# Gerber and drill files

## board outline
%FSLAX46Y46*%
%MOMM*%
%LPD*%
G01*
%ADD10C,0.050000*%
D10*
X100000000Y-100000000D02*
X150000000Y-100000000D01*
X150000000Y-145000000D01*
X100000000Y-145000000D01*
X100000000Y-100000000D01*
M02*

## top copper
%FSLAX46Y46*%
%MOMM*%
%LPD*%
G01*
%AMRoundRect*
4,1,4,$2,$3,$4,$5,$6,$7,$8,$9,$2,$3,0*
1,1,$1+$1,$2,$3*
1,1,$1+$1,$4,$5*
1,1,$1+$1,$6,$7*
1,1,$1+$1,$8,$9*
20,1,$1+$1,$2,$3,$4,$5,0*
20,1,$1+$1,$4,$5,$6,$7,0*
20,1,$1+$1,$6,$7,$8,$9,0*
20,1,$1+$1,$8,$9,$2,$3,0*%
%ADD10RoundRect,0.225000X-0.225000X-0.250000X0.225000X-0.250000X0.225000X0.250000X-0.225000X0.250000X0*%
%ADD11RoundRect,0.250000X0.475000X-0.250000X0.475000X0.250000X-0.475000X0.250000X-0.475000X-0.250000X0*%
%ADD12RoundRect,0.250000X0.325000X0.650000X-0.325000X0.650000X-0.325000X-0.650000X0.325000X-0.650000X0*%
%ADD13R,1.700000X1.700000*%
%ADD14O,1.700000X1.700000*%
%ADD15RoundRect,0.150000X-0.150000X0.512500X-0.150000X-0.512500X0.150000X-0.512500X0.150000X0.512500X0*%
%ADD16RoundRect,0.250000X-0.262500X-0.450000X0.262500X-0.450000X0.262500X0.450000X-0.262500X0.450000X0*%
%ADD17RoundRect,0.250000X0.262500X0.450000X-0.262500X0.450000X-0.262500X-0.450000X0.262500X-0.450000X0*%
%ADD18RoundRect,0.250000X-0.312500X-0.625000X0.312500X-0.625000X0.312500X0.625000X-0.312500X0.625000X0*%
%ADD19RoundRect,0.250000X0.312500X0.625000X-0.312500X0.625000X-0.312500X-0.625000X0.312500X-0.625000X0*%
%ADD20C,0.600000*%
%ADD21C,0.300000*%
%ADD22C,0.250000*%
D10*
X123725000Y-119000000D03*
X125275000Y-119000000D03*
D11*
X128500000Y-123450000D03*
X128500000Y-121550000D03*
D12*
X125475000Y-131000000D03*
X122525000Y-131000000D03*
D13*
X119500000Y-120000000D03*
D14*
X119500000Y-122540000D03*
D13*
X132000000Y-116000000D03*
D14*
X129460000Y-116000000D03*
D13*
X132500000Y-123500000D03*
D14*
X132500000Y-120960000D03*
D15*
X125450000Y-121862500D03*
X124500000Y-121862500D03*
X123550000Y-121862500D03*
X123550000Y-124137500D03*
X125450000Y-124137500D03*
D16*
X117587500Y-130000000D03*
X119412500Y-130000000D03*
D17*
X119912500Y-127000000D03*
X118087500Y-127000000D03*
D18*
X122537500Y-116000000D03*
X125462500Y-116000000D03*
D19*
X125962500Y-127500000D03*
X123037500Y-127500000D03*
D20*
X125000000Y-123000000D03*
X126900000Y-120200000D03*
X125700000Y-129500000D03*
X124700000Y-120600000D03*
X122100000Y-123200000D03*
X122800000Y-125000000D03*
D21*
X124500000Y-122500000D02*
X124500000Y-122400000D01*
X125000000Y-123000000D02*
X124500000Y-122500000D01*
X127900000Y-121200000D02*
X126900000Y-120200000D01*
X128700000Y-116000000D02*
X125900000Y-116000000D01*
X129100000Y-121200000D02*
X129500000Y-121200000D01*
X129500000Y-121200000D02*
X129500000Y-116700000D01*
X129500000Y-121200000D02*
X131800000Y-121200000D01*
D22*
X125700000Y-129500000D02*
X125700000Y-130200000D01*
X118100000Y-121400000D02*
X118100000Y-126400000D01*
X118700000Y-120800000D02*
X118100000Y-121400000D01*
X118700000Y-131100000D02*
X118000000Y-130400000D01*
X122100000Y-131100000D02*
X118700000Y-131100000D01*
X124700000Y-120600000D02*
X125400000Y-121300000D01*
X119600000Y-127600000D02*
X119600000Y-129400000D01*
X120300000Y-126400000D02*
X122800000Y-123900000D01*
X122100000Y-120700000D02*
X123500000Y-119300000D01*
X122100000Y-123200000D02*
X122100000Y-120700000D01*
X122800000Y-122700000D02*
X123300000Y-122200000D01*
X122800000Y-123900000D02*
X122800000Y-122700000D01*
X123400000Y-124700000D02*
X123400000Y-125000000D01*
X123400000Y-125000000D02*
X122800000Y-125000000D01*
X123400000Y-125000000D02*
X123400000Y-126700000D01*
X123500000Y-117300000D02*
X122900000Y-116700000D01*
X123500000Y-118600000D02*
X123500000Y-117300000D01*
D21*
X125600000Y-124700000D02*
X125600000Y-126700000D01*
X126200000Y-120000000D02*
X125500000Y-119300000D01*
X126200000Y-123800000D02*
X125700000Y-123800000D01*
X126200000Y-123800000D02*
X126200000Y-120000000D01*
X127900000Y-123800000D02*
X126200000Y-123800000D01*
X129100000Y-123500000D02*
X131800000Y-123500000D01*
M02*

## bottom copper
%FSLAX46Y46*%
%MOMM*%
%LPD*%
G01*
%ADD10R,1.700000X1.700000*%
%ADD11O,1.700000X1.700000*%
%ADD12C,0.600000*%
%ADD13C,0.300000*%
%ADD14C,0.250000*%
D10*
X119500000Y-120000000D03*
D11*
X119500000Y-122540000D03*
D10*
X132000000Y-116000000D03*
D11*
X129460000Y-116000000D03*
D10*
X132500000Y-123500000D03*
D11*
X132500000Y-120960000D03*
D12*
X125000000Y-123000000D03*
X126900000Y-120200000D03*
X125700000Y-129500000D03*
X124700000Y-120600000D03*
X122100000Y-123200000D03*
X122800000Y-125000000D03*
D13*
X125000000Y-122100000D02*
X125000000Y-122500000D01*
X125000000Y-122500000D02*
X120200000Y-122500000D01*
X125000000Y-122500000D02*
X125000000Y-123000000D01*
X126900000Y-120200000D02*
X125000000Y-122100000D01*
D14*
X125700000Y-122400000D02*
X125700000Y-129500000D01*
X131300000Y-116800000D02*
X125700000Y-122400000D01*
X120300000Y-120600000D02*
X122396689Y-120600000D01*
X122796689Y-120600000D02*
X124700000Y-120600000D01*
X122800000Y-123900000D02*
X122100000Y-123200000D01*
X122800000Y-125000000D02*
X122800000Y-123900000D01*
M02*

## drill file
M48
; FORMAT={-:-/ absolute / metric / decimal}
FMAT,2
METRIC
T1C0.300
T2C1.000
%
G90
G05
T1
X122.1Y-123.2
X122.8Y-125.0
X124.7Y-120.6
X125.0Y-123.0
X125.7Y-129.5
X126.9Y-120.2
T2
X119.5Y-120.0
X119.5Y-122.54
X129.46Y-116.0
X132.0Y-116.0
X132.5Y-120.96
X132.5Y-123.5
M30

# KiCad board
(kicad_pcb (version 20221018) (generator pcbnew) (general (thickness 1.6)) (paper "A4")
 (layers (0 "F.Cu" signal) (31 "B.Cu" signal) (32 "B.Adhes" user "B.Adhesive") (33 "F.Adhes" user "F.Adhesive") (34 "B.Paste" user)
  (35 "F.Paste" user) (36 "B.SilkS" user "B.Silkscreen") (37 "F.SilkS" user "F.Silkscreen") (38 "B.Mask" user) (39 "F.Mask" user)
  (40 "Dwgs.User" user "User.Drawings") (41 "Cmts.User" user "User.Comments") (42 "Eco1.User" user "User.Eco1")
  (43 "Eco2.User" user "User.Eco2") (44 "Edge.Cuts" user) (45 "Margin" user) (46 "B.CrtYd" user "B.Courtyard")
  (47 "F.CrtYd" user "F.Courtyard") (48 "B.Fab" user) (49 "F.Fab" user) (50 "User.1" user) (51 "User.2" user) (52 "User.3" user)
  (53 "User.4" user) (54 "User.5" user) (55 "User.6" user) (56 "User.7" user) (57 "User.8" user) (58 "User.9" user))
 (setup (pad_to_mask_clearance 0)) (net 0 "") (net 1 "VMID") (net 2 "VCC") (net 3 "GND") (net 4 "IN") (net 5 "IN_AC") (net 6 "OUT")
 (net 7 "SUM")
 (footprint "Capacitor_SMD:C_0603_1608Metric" (layer "F.Cu") (at 124.5 119)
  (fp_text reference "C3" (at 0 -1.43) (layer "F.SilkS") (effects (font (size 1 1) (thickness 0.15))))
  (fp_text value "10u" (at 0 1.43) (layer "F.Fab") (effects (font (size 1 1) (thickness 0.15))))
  (pad "1" smd roundrect (at -0.775 0) (size 0.9 0.95) (layers "F.Cu" "F.Paste" "F.Mask") (roundrect_rratio 0.25) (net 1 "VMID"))
  (pad "2" smd roundrect (at 0.775 0) (size 0.9 0.95) (layers "F.Cu" "F.Paste" "F.Mask") (roundrect_rratio 0.25) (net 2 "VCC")))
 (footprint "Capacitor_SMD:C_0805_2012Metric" (layer "F.Cu") (at 128.5 122.5 90)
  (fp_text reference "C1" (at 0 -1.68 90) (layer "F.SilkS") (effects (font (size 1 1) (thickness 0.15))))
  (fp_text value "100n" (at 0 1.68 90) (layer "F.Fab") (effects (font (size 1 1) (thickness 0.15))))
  (pad "1" smd roundrect (at -0.95 0 90) (size 1 1.45) (layers "F.Cu" "F.Paste" "F.Mask") (roundrect_rratio 0.25) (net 2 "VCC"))
  (pad "2" smd roundrect (at 0.95 0 90) (size 1 1.45) (layers "F.Cu" "F.Paste" "F.Mask") (roundrect_rratio 0.25) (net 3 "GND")))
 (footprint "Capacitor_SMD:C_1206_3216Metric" (layer "F.Cu") (at 124 131 180)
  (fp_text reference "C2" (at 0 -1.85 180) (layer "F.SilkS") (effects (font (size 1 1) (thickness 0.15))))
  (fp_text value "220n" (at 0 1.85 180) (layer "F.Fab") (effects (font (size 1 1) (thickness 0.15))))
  (pad "1" smd roundrect (at -1.475 0 180) (size 1.15 1.8) (layers "F.Cu" "F.Paste" "F.Mask") (roundrect_rratio 0.217391) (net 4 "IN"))
  (pad "2" smd roundrect (at 1.475 0 180) (size 1.15 1.8) (layers "F.Cu" "F.Paste" "F.Mask") (roundrect_rratio 0.217391) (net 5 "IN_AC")))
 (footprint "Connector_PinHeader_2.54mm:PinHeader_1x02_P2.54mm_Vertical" (layer "F.Cu") (at 119.5 120)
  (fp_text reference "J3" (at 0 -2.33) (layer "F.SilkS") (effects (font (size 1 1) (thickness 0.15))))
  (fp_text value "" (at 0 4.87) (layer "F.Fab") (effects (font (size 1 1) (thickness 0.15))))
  (pad "1" thru_hole rect (at 0 0) (size 1.7 1.7) (drill 1) (layers "*.Cu" "*.Mask") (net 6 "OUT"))
  (pad "2" thru_hole oval (at 0 2.54) (size 1.7 1.7) (drill 1) (layers "*.Cu" "*.Mask") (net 3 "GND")))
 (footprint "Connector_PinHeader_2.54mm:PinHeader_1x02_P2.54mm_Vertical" (layer "F.Cu") (at 132 116 -90)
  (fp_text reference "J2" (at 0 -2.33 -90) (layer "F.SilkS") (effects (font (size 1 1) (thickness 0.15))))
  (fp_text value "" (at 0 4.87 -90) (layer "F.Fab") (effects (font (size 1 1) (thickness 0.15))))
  (pad "1" thru_hole rect (at 0 0 270) (size 1.7 1.7) (drill 1) (layers "*.Cu" "*.Mask") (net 4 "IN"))
  (pad "2" thru_hole oval (at 0 2.54 270) (size 1.7 1.7) (drill 1) (layers "*.Cu" "*.Mask") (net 3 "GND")))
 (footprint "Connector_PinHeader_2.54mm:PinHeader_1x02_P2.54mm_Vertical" (layer "F.Cu") (at 132.5 123.5 180)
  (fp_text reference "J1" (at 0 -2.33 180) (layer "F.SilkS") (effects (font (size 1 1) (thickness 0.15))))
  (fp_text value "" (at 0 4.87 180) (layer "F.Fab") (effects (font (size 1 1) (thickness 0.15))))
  (pad "1" thru_hole rect (at 0 0 180) (size 1.7 1.7) (drill 1) (layers "*.Cu" "*.Mask") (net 2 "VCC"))
  (pad "2" thru_hole oval (at 0 2.54 180) (size 1.7 1.7) (drill 1) (layers "*.Cu" "*.Mask") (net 3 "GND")))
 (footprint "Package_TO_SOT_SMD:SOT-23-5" (layer "F.Cu") (at 124.5 123 -90)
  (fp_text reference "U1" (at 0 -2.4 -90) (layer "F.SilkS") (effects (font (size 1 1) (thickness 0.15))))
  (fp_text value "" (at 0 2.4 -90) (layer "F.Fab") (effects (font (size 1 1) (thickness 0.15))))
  (pad "1" smd roundrect (at -1.1375 -0.95 270) (size 1.325 0.6) (layers "F.Cu" "F.Paste" "F.Mask") (roundrect_rratio 0.25) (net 6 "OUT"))
  (pad "2" smd roundrect (at -1.1375 0 270) (size 1.325 0.6) (layers "F.Cu" "F.Paste" "F.Mask") (roundrect_rratio 0.25) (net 3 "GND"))
  (pad "3" smd roundrect (at -1.1375 0.95 270) (size 1.325 0.6) (layers "F.Cu" "F.Paste" "F.Mask") (roundrect_rratio 0.25) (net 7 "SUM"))
  (pad "4" smd roundrect (at 1.1375 0.95 270) (size 1.325 0.6) (layers "F.Cu" "F.Paste" "F.Mask") (roundrect_rratio 0.25) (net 1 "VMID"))
  (pad "5" smd roundrect (at 1.1375 -0.95 270) (size 1.325 0.6) (layers "F.Cu" "F.Paste" "F.Mask") (roundrect_rratio 0.25) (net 2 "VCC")))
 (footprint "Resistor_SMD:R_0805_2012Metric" (layer "F.Cu") (at 118.5 130)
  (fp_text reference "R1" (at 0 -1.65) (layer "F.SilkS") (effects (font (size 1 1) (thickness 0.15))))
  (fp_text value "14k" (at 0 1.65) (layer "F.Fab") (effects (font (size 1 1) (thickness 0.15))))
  (pad "1" smd roundrect (at -0.9125 0) (size 1.025 1.4) (layers "F.Cu" "F.Paste" "F.Mask") (roundrect_rratio 0.243902) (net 5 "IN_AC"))
  (pad "2" smd roundrect (at 0.9125 0) (size 1.025 1.4) (layers "F.Cu" "F.Paste" "F.Mask") (roundrect_rratio 0.243902) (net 7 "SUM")))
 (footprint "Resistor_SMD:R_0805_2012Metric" (layer "F.Cu") (at 119 127 180)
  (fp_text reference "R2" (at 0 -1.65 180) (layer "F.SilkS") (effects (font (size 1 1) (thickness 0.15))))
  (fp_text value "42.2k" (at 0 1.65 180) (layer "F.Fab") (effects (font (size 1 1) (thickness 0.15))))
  (pad "1" smd roundrect (at -0.9125 0 180) (size 1.025 1.4) (layers "F.Cu" "F.Paste" "F.Mask") (roundrect_rratio 0.243902) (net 7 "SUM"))
  (pad "2" smd roundrect (at 0.9125 0 180) (size 1.025 1.4) (layers "F.Cu" "F.Paste" "F.Mask") (roundrect_rratio 0.243902) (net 6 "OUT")))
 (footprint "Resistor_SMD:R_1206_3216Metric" (layer "F.Cu") (at 124 116)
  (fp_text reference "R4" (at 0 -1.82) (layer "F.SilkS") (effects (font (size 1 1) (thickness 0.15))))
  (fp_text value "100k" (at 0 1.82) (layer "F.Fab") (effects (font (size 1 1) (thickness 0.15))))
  (pad "1" smd roundrect (at -1.4625 0) (size 1.125 1.75) (layers "F.Cu" "F.Paste" "F.Mask") (roundrect_rratio 0.222222) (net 1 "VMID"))
  (pad "2" smd roundrect (at 1.4625 0) (size 1.125 1.75) (layers "F.Cu" "F.Paste" "F.Mask") (roundrect_rratio 0.222222) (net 3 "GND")))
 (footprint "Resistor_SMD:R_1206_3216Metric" (layer "F.Cu") (at 124.5 127.5 180)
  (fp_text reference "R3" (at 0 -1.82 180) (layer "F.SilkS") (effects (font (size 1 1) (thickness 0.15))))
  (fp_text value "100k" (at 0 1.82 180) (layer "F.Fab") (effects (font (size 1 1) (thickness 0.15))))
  (pad "1" smd roundrect (at -1.4625 0 180) (size 1.125 1.75) (layers "F.Cu" "F.Paste" "F.Mask") (roundrect_rratio 0.222222) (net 2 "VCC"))
  (pad "2" smd roundrect (at 1.4625 0 180) (size 1.125 1.75) (layers "F.Cu" "F.Paste" "F.Mask") (roundrect_rratio 0.222222) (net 1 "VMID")))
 (gr_rect (start 100 100) (end 150 145) (stroke (width 0.05) (type default)) (fill none) (layer "Edge.Cuts"))
 (segment (start 124.5 122.5) (end 124.5 122.4) (width 0.3) (layer "F.Cu") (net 3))
 (segment (start 125 123) (end 124.5 122.5) (width 0.3) (layer "F.Cu") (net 3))
 (segment (start 127.9 121.2) (end 126.9 120.2) (width 0.3) (layer "F.Cu") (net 3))
 (segment (start 128.7 116) (end 125.9 116) (width 0.3) (layer "F.Cu") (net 3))
 (segment (start 129.1 121.2) (end 129.5 121.2) (width 0.3) (layer "F.Cu") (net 3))
 (segment (start 129.5 121.2) (end 129.5 116.7) (width 0.3) (layer "F.Cu") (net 3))
 (segment (start 129.5 121.2) (end 131.8 121.2) (width 0.3) (layer "F.Cu") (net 3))
 (via (at 125 123) (size 0.6) (drill 0.3) (layers "F.Cu" "B.Cu") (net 3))
 (via (at 126.9 120.2) (size 0.6) (drill 0.3) (layers "F.Cu" "B.Cu") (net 3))
 (segment (start 125 122.1) (end 125 122.5) (width 0.3) (layer "B.Cu") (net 3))
 (segment (start 125 122.5) (end 120.2 122.5) (width 0.3) (layer "B.Cu") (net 3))
 (segment (start 125 122.5) (end 125 123) (width 0.3) (layer "B.Cu") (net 3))
 (segment (start 125.7 129.5) (end 125.7 130.2) (width 0.25) (layer "F.Cu") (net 4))
 (segment (start 126.9 120.2) (end 125 122.1) (width 0.3) (layer "B.Cu") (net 3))
 (via (at 125.7 129.5) (size 0.6) (drill 0.3) (layers "F.Cu" "B.Cu") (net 4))
 (segment (start 118.1 121.4) (end 118.1 126.4) (width 0.25) (layer "F.Cu") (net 6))
 (segment (start 118.7 120.8) (end 118.1 121.4) (width 0.25) (layer "F.Cu") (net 6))
 (segment (start 118.7 131.1) (end 118 130.4) (width 0.25) (layer "F.Cu") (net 5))
 (segment (start 122.1 131.1) (end 118.7 131.1) (width 0.25) (layer "F.Cu") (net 5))
 (segment (start 124.7 120.6) (end 125.4 121.3) (width 0.25) (layer "F.Cu") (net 6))
 (segment (start 125.7 122.4) (end 125.7 129.5) (width 0.25) (layer "B.Cu") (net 4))
 (segment (start 131.3 116.8) (end 125.7 122.4) (width 0.25) (layer "B.Cu") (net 4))
 (via (at 124.7 120.6) (size 0.6) (drill 0.3) (layers "F.Cu" "B.Cu") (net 6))
 (segment (start 119.6 127.6) (end 119.6 129.4) (width 0.25) (layer "F.Cu") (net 7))
 (segment (start 120.3 120.6) (end 122.396689 120.6) (width 0.25) (layer "B.Cu") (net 6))
 (segment (start 120.3 126.4) (end 122.8 123.9) (width 0.25) (layer "F.Cu") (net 7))
 (segment (start 122.1 120.7) (end 123.5 119.3) (width 0.25) (layer "F.Cu") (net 1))
 (segment (start 122.1 123.2) (end 122.1 120.7) (width 0.25) (layer "F.Cu") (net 1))
 (segment (start 122.796689 120.6) (end 124.7 120.6) (width 0.25) (layer "B.Cu") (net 6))
 (segment (start 122.8 122.7) (end 123.3 122.2) (width 0.25) (layer "F.Cu") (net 7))
 (segment (start 122.8 123.9) (end 122.8 122.7) (width 0.25) (layer "F.Cu") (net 7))
 (segment (start 123.4 124.7) (end 123.4 125) (width 0.25) (layer "F.Cu") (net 1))
 (segment (start 123.4 125) (end 122.8 125) (width 0.25) (layer "F.Cu") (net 1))
 (segment (start 123.4 125) (end 123.4 126.7) (width 0.25) (layer "F.Cu") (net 1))
 (segment (start 123.5 117.3) (end 122.9 116.7) (width 0.25) (layer "F.Cu") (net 1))
 (segment (start 123.5 118.6) (end 123.5 117.3) (width 0.25) (layer "F.Cu") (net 1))
 (segment (start 125.6 124.7) (end 125.6 126.7) (width 0.3) (layer "F.Cu") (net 2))
 (segment (start 126.2 120) (end 125.5 119.3) (width 0.3) (layer "F.Cu") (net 2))
 (segment (start 126.2 123.8) (end 125.7 123.8) (width 0.3) (layer "F.Cu") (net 2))
 (segment (start 126.2 123.8) (end 126.2 120) (width 0.3) (layer "F.Cu") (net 2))
 (segment (start 127.9 123.8) (end 126.2 123.8) (width 0.3) (layer "F.Cu") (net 2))
 (segment (start 129.1 123.5) (end 131.8 123.5) (width 0.3) (layer "F.Cu") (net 2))
 (via (at 122.1 123.2) (size 0.6) (drill 0.3) (layers "F.Cu" "B.Cu") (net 1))
 (via (at 122.8 125) (size 0.6) (drill 0.3) (layers "F.Cu" "B.Cu") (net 1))
 (segment (start 122.8 123.9) (end 122.1 123.2) (width 0.25) (layer "B.Cu") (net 1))
 (segment (start 122.8 125) (end 122.8 123.9) (width 0.25) (layer "B.Cu") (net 1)))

